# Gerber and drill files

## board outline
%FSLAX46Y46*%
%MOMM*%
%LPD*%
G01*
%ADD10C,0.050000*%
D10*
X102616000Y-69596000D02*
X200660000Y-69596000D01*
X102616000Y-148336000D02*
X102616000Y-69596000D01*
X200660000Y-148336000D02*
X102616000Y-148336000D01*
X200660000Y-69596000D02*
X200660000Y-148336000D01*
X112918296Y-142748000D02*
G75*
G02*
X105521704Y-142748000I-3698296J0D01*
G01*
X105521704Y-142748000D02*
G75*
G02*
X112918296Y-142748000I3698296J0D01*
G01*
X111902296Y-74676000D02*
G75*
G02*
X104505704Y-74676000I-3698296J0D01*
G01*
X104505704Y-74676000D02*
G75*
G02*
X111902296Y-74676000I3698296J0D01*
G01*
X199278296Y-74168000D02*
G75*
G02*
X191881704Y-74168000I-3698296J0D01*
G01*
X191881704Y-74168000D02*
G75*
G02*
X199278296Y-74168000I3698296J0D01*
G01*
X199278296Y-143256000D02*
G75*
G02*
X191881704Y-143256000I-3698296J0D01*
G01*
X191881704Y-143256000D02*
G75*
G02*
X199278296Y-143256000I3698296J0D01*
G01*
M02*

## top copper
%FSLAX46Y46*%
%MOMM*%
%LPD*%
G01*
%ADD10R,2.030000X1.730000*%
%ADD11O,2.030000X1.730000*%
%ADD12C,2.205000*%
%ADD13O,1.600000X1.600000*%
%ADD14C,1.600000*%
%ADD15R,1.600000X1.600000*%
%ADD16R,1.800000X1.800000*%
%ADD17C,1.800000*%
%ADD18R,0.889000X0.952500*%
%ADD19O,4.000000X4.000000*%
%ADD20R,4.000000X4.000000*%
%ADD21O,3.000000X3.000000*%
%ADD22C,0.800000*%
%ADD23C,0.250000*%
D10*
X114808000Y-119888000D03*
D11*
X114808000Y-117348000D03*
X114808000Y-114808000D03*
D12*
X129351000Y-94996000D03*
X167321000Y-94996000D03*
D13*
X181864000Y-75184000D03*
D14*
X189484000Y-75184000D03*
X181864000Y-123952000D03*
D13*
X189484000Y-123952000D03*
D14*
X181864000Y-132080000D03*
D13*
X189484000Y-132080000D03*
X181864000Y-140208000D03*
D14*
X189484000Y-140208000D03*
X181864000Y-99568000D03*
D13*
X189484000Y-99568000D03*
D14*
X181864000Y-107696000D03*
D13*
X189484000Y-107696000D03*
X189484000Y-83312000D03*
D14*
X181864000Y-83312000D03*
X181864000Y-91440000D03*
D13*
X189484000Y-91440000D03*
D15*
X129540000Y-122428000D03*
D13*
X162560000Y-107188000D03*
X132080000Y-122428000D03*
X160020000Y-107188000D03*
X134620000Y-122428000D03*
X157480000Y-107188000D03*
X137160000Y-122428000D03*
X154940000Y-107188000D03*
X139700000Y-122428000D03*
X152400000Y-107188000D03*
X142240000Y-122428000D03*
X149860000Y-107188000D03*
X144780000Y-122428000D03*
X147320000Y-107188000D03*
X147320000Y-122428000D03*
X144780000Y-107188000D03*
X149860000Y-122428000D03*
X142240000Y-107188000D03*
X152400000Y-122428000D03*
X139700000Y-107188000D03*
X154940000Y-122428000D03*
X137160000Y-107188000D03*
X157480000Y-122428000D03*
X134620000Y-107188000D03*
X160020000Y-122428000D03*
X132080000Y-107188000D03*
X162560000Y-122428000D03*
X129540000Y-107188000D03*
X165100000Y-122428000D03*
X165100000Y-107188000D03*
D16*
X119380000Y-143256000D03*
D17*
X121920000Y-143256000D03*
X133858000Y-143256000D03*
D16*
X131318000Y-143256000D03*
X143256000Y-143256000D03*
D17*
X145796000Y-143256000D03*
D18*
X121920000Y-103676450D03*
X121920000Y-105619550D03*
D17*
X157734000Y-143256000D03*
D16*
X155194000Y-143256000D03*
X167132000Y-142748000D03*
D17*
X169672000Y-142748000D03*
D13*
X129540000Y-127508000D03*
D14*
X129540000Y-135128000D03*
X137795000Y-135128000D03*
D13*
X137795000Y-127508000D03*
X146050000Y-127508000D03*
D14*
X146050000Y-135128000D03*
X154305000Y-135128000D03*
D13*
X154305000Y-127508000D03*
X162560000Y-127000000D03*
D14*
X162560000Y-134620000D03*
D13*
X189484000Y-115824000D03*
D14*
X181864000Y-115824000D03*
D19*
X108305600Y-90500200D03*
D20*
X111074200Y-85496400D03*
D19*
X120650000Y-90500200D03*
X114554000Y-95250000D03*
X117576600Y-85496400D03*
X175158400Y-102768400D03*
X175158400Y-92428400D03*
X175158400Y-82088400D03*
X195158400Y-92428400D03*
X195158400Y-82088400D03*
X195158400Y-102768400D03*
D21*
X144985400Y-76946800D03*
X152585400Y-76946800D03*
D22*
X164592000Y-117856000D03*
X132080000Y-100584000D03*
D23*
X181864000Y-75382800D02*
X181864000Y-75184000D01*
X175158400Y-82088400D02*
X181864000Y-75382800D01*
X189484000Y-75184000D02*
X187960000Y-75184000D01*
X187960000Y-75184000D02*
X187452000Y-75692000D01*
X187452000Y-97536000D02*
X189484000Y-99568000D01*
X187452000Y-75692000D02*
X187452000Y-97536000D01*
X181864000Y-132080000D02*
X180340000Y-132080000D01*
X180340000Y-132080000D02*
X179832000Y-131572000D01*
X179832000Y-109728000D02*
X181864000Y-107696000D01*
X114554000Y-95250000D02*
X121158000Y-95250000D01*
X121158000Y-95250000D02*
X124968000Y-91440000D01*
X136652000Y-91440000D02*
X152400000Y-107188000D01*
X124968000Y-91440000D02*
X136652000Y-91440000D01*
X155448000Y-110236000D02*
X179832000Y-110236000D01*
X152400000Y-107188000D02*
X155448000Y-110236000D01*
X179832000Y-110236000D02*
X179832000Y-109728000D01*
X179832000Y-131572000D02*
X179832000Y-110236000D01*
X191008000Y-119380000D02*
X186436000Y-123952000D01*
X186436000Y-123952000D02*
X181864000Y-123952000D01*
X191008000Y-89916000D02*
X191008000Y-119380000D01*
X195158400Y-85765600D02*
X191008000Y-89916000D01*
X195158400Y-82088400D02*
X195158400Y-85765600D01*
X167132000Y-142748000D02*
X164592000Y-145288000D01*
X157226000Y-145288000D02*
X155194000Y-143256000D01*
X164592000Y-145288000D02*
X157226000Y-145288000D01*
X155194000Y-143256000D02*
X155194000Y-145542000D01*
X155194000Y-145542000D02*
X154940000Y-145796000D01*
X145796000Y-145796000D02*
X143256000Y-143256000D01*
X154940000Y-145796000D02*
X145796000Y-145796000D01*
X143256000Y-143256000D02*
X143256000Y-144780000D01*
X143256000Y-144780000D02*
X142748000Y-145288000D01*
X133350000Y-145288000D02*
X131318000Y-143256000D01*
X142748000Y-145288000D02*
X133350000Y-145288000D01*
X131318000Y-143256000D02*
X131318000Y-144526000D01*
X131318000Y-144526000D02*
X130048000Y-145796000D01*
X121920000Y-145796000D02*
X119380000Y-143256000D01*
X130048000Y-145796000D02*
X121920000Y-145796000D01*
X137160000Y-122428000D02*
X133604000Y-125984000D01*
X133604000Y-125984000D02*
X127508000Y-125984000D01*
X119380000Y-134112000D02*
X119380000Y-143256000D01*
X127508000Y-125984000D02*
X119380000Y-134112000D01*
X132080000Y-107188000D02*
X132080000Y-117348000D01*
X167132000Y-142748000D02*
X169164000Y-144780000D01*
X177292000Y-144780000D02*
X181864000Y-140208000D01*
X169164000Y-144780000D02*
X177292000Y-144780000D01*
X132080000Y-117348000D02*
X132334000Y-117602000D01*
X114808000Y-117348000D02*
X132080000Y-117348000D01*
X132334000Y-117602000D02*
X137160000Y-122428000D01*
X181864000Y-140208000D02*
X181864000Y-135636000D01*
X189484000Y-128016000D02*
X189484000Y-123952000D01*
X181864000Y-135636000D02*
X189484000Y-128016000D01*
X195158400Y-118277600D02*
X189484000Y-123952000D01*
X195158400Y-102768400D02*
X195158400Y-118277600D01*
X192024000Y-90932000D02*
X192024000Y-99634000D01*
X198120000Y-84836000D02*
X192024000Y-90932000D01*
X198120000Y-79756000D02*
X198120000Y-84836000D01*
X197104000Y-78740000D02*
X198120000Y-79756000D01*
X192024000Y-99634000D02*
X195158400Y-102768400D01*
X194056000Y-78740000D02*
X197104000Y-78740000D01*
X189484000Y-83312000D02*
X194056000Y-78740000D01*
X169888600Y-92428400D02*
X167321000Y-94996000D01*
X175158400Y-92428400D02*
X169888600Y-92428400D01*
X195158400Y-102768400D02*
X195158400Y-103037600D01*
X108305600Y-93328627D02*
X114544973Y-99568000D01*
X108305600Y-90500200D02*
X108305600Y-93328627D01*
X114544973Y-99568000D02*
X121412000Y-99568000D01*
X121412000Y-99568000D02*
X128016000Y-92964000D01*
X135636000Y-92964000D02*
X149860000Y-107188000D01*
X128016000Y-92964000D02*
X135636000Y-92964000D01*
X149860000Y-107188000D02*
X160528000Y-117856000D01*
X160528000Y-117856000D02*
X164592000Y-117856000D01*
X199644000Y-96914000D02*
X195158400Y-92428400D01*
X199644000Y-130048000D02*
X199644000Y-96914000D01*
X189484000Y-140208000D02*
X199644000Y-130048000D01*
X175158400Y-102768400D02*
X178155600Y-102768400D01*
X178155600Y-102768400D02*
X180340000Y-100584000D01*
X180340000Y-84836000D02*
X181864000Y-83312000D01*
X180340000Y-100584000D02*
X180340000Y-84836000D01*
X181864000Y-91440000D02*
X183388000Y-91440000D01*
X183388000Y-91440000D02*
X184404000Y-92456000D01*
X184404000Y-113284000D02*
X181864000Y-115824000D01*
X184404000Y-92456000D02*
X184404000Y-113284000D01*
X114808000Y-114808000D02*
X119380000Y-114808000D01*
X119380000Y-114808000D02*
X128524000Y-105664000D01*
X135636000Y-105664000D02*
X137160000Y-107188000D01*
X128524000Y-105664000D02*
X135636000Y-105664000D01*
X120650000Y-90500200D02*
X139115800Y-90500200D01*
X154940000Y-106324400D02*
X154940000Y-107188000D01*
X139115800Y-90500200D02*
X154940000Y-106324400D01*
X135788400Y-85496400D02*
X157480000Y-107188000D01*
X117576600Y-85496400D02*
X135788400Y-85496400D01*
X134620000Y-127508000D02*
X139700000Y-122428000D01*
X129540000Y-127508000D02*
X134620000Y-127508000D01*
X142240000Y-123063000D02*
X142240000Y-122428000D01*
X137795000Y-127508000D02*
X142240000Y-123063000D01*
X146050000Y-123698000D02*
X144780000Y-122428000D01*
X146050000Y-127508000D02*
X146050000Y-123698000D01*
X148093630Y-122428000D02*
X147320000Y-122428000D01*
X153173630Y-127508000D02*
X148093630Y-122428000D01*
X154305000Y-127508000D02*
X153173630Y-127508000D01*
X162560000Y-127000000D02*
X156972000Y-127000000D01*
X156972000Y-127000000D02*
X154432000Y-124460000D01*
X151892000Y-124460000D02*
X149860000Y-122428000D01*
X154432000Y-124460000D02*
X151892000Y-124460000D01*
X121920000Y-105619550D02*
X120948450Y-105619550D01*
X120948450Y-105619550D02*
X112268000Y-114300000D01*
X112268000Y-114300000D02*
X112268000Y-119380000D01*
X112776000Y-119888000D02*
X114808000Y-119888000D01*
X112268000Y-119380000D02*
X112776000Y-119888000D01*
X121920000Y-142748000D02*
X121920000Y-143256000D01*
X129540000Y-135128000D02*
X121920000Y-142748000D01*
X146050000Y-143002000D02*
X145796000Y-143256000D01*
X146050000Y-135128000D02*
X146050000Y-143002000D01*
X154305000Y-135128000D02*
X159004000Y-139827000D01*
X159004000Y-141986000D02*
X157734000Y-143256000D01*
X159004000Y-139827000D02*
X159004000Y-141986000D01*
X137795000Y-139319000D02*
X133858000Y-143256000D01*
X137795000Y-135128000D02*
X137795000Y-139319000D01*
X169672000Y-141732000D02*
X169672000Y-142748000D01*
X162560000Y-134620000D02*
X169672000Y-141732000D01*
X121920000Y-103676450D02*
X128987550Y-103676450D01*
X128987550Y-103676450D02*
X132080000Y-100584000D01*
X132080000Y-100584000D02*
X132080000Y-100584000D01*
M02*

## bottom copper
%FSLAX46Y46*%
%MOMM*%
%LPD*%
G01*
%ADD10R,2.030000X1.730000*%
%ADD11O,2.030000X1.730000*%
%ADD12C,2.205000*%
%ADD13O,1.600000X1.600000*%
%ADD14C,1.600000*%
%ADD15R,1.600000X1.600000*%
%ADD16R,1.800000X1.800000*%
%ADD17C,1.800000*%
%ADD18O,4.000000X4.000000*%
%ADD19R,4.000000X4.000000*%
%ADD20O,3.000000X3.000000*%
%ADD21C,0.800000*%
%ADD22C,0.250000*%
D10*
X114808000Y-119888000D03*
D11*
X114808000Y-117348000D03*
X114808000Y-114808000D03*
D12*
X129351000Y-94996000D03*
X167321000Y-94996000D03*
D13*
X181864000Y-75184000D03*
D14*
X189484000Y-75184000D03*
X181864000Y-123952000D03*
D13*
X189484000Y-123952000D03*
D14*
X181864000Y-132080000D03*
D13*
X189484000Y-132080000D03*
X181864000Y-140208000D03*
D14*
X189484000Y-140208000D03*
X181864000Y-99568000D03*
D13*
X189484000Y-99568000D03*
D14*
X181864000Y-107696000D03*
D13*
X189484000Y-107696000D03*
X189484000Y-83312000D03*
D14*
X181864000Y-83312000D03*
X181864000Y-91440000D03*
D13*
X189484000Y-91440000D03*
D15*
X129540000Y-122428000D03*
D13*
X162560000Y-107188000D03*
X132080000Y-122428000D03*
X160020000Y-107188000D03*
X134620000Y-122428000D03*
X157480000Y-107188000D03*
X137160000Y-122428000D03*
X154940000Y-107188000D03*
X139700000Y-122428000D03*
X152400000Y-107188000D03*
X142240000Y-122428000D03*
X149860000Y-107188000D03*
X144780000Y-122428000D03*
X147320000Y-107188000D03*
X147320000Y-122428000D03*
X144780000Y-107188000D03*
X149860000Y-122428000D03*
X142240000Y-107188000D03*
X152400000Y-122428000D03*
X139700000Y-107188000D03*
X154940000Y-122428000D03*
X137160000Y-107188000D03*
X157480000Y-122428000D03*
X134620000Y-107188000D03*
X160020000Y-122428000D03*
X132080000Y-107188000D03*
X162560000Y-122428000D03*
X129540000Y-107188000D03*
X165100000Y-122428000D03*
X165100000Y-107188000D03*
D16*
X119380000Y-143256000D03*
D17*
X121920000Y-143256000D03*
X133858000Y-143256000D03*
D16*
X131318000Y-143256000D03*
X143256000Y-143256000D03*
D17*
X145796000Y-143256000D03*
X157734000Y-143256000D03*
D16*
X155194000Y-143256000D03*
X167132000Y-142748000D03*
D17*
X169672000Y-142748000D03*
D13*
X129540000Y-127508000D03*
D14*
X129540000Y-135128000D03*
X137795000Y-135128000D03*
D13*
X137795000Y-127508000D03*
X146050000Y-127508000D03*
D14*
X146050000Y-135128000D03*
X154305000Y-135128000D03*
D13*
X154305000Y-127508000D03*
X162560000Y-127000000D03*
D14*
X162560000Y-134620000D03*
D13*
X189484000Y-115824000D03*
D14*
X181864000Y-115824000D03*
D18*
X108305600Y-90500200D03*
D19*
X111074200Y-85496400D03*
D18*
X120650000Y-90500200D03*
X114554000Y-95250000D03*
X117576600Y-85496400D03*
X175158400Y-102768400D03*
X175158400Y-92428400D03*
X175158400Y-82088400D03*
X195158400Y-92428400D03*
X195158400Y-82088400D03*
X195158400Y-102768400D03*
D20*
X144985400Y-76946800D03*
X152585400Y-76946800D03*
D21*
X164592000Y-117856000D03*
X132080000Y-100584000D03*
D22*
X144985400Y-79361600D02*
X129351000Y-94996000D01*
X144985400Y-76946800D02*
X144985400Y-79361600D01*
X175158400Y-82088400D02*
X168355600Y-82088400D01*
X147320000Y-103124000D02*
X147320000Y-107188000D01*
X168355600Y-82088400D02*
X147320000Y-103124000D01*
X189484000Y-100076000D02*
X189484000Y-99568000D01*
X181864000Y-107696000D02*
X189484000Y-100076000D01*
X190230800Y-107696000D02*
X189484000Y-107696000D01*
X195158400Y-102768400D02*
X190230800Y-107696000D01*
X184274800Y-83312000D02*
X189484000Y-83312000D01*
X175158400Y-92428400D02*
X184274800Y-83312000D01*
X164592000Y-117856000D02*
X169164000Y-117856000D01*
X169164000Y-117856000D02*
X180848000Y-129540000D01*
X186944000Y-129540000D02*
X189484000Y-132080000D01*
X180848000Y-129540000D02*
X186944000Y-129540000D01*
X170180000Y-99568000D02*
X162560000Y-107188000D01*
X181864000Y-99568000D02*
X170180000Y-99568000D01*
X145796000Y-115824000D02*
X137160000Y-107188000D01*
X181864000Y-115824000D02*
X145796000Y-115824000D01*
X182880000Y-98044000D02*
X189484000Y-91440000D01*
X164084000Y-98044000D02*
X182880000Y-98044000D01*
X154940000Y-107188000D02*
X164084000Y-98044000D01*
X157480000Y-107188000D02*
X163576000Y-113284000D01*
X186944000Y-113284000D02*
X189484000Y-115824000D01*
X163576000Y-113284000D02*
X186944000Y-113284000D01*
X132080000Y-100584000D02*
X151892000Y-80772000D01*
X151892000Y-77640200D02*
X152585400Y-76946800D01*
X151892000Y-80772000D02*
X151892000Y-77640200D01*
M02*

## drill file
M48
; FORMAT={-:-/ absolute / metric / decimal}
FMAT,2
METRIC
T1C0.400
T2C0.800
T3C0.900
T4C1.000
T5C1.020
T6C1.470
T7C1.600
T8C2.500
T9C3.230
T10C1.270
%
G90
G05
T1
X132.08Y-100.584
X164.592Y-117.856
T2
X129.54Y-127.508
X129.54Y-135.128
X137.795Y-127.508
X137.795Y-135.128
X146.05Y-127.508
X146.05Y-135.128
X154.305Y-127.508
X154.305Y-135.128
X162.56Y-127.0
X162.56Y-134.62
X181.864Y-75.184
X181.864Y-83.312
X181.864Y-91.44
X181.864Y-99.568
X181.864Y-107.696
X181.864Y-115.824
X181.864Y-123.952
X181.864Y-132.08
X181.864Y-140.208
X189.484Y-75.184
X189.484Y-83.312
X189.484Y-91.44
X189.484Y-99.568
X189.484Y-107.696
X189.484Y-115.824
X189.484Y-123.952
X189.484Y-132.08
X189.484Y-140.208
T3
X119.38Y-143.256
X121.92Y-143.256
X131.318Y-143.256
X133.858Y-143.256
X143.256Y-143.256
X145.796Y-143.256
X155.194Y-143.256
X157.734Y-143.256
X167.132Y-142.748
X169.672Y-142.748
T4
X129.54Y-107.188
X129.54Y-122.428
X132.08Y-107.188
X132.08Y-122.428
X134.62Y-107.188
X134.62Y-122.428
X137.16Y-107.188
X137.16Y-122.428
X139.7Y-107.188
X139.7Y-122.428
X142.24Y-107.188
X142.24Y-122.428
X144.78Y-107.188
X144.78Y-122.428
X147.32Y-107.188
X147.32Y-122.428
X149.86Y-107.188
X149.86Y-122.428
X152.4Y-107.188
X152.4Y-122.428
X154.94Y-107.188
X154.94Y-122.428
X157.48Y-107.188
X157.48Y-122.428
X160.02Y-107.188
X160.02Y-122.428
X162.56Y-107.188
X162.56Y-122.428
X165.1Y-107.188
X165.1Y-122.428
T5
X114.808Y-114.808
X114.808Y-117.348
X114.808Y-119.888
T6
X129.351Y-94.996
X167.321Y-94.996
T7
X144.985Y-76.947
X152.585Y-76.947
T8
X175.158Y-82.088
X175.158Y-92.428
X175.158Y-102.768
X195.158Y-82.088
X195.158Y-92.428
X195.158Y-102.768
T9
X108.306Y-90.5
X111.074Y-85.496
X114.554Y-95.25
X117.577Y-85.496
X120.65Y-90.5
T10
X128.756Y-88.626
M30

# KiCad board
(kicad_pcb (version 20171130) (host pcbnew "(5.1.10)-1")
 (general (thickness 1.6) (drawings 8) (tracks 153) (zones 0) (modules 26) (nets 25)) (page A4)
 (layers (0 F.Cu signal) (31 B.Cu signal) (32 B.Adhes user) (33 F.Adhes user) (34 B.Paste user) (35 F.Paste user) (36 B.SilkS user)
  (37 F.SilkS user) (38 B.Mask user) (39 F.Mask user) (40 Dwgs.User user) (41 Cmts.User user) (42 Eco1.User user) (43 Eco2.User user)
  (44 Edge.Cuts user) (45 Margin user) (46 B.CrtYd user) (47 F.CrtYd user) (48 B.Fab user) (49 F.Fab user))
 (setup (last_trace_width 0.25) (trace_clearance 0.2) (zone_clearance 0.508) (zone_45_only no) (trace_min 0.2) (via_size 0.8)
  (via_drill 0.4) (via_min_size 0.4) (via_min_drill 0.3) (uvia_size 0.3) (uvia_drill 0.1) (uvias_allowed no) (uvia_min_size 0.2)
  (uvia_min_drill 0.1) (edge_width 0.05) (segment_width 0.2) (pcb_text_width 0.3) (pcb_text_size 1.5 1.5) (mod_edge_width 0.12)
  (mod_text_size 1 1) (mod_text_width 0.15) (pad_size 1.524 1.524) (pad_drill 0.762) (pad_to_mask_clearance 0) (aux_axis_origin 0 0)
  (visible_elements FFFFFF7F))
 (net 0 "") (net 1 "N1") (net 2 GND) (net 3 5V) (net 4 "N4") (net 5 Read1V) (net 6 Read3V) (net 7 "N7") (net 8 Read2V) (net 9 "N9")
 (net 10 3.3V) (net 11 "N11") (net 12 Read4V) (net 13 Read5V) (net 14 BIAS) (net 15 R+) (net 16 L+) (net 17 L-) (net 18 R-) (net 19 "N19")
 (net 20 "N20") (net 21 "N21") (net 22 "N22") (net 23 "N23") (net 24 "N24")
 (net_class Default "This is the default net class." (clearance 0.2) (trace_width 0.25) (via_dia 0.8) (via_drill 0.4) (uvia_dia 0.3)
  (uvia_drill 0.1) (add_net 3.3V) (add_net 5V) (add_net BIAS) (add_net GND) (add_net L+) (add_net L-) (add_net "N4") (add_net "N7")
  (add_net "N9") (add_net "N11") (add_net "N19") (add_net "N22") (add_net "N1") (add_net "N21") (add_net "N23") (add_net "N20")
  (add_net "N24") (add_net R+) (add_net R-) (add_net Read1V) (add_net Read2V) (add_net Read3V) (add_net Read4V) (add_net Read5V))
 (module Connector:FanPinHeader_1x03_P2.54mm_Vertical (layer F.Cu) (at 114.808 119.888 90)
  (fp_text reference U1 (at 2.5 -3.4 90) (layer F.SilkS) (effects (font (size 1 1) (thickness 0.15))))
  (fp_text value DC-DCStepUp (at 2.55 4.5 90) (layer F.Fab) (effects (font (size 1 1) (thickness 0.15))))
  (pad 1 thru_hole rect (at 0 0 180) (size 2.03 1.73) (drill 1.02) (layers *.Cu *.Mask) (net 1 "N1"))
  (pad 3 thru_hole oval (at 2.54 0 180) (size 2.03 1.73) (drill 1.02) (layers *.Cu *.Mask) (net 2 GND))
  (pad 2 thru_hole oval (at 5.08 0 180) (size 2.03 1.73) (drill 1.02) (layers *.Cu *.Mask) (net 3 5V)))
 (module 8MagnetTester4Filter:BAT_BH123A (layer F.Cu) (at 148.336 94.996 180)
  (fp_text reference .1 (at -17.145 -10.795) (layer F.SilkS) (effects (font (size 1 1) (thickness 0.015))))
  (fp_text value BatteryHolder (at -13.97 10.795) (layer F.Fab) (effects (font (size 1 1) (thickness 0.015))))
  (pad None np_thru_hole circle (at 19.58 6.37 180) (size 1.27 1.27) (drill 1.27) (layers *.Cu *.Mask))
  (pad 2 thru_hole circle (at 18.985 0 180) (size 2.205 2.205) (drill 1.47) (layers *.Cu *.Mask) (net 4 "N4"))
  (pad 1 thru_hole circle (at -18.985 0 180) (size 2.205 2.205) (drill 1.47) (layers *.Cu *.Mask) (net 2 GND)))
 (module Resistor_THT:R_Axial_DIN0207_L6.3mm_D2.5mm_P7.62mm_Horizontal (layer F.Cu) (at 189.484 75.184 180)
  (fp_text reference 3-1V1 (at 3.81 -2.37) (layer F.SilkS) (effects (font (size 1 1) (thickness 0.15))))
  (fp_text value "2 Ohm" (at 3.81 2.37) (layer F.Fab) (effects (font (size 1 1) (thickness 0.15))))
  (pad 2 thru_hole oval (at 7.62 0 180) (size 1.6 1.6) (drill 0.8) (layers *.Cu *.Mask) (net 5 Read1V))
  (pad 1 thru_hole circle (at 0 0 180) (size 1.6 1.6) (drill 0.8) (layers *.Cu *.Mask) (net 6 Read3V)))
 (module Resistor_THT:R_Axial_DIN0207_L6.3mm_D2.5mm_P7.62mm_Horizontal (layer F.Cu) (at 181.864 123.952)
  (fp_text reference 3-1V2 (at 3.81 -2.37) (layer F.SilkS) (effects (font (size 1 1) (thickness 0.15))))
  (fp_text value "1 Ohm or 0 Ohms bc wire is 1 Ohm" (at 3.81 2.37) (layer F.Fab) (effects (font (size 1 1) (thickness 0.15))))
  (pad 1 thru_hole circle (at 0 0) (size 1.6 1.6) (drill 0.8) (layers *.Cu *.Mask) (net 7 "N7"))
  (pad 2 thru_hole oval (at 7.62 0) (size 1.6 1.6) (drill 0.8) (layers *.Cu *.Mask) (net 2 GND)))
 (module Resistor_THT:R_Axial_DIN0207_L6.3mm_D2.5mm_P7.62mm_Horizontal (layer F.Cu) (at 181.864 132.08)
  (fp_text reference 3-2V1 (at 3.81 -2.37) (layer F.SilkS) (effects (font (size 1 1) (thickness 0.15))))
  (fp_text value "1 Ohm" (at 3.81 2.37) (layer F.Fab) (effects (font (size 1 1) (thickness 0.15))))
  (pad 1 thru_hole circle (at 0 0) (size 1.6 1.6) (drill 0.8) (layers *.Cu *.Mask) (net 6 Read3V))
  (pad 2 thru_hole oval (at 7.62 0) (size 1.6 1.6) (drill 0.8) (layers *.Cu *.Mask) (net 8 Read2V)))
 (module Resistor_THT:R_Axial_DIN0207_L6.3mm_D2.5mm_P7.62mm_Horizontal (layer F.Cu) (at 189.484 140.208 180)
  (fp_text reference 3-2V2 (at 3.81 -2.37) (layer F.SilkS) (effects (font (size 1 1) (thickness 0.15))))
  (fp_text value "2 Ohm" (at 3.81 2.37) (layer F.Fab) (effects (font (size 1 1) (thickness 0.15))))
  (pad 2 thru_hole oval (at 7.62 0 180) (size 1.6 1.6) (drill 0.8) (layers *.Cu *.Mask) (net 2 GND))
  (pad 1 thru_hole circle (at 0 0 180) (size 1.6 1.6) (drill 0.8) (layers *.Cu *.Mask) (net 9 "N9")))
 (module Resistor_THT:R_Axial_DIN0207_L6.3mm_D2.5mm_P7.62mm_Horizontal (layer F.Cu) (at 181.864 99.568)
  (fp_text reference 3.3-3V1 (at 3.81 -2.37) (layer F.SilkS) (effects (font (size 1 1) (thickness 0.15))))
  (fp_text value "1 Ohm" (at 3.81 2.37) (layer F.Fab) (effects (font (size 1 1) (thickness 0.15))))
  (pad 1 thru_hole circle (at 0 0) (size 1.6 1.6) (drill 0.8) (layers *.Cu *.Mask) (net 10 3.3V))
  (pad 2 thru_hole oval (at 7.62 0) (size 1.6 1.6) (drill 0.8) (layers *.Cu *.Mask) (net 6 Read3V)))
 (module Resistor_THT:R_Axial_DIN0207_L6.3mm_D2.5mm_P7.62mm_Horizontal (layer F.Cu) (at 181.864 107.696)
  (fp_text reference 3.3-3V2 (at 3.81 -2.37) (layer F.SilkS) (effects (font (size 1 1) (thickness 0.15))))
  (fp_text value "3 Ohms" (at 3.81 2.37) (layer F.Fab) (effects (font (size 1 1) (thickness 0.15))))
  (pad 1 thru_hole circle (at 0 0) (size 1.6 1.6) (drill 0.8) (layers *.Cu *.Mask) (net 6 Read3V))
  (pad 2 thru_hole oval (at 7.62 0) (size 1.6 1.6) (drill 0.8) (layers *.Cu *.Mask) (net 2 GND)))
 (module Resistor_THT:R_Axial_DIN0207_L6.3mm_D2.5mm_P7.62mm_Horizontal (layer F.Cu) (at 181.864 83.312)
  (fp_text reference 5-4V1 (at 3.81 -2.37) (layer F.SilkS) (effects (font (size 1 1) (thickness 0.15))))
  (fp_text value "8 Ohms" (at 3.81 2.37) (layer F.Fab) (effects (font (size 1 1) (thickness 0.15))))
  (pad 2 thru_hole oval (at 7.62 0) (size 1.6 1.6) (drill 0.8) (layers *.Cu *.Mask) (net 2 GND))
  (pad 1 thru_hole circle (at 0 0) (size 1.6 1.6) (drill 0.8) (layers *.Cu *.Mask) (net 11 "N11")))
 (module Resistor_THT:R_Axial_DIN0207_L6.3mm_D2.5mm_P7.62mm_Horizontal (layer F.Cu) (at 181.864 91.44)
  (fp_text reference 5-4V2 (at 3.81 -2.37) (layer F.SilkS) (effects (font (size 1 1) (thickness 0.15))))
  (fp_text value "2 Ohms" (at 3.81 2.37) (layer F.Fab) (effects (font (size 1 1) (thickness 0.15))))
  (pad 1 thru_hole circle (at 0 0) (size 1.6 1.6) (drill 0.8) (layers *.Cu *.Mask) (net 3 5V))
  (pad 2 thru_hole oval (at 7.62 0) (size 1.6 1.6) (drill 0.8) (layers *.Cu *.Mask) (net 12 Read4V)))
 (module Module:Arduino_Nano (layer F.Cu) (at 129.54 122.428 90)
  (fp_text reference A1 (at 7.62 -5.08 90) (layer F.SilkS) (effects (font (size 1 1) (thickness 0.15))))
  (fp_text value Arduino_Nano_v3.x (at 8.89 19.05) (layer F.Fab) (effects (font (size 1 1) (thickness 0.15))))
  (pad 1 thru_hole rect (at 0 0 90) (size 1.6 1.6) (drill 1) (layers *.Cu *.Mask))
  (pad 17 thru_hole oval (at 15.24 33.02 90) (size 1.6 1.6) (drill 1) (layers *.Cu *.Mask) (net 10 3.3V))
  (pad 2 thru_hole oval (at 0 2.54 90) (size 1.6 1.6) (drill 1) (layers *.Cu *.Mask))
  (pad 18 thru_hole oval (at 15.24 30.48 90) (size 1.6 1.6) (drill 1) (layers *.Cu *.Mask))
  (pad 3 thru_hole oval (at 0 5.08 90) (size 1.6 1.6) (drill 1) (layers *.Cu *.Mask))
  (pad 19 thru_hole oval (at 15.24 27.94 90) (size 1.6 1.6) (drill 1) (layers *.Cu *.Mask) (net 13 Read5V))
  (pad 4 thru_hole oval (at 0 7.62 90) (size 1.6 1.6) (drill 1) (layers *.Cu *.Mask) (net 2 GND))
  (pad 20 thru_hole oval (at 15.24 25.4 90) (size 1.6 1.6) (drill 1) (layers *.Cu *.Mask) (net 12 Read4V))
  (pad 5 thru_hole oval (at 0 10.16 90) (size 1.6 1.6) (drill 1) (layers *.Cu *.Mask) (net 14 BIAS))
  (pad 21 thru_hole oval (at 15.24 22.86 90) (size 1.6 1.6) (drill 1) (layers *.Cu *.Mask) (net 6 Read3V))
  (pad 6 thru_hole oval (at 0 12.7 90) (size 1.6 1.6) (drill 1) (layers *.Cu *.Mask) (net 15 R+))
  (pad 22 thru_hole oval (at 15.24 20.32 90) (size 1.6 1.6) (drill 1) (layers *.Cu *.Mask) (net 8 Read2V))
  (pad 7 thru_hole oval (at 0 15.24 90) (size 1.6 1.6) (drill 1) (layers *.Cu *.Mask) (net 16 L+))
  (pad 23 thru_hole oval (at 15.24 17.78 90) (size 1.6 1.6) (drill 1) (layers *.Cu *.Mask) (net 5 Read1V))
  (pad 8 thru_hole oval (at 0 17.78 90) (size 1.6 1.6) (drill 1) (layers *.Cu *.Mask) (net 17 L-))
  (pad 24 thru_hole oval (at 15.24 15.24 90) (size 1.6 1.6) (drill 1) (layers *.Cu *.Mask))
  (pad 9 thru_hole oval (at 0 20.32 90) (size 1.6 1.6) (drill 1) (layers *.Cu *.Mask) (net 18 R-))
  (pad 25 thru_hole oval (at 15.24 12.7 90) (size 1.6 1.6) (drill 1) (layers *.Cu *.Mask))
  (pad 10 thru_hole oval (at 0 22.86 90) (size 1.6 1.6) (drill 1) (layers *.Cu *.Mask))
  (pad 26 thru_hole oval (at 15.24 10.16 90) (size 1.6 1.6) (drill 1) (layers *.Cu *.Mask))
  (pad 11 thru_hole oval (at 0 25.4 90) (size 1.6 1.6) (drill 1) (layers *.Cu *.Mask))
  (pad 27 thru_hole oval (at 15.24 7.62 90) (size 1.6 1.6) (drill 1) (layers *.Cu *.Mask) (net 3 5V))
  (pad 12 thru_hole oval (at 0 27.94 90) (size 1.6 1.6) (drill 1) (layers *.Cu *.Mask))
  (pad 28 thru_hole oval (at 15.24 5.08 90) (size 1.6 1.6) (drill 1) (layers *.Cu *.Mask))
  (pad 13 thru_hole oval (at 0 30.48 90) (size 1.6 1.6) (drill 1) (layers *.Cu *.Mask))
  (pad 29 thru_hole oval (at 15.24 2.54 90) (size 1.6 1.6) (drill 1) (layers *.Cu *.Mask) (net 2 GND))
  (pad 14 thru_hole oval (at 0 33.02 90) (size 1.6 1.6) (drill 1) (layers *.Cu *.Mask))
  (pad 30 thru_hole oval (at 15.24 0 90) (size 1.6 1.6) (drill 1) (layers *.Cu *.Mask))
  (pad 15 thru_hole oval (at 0 35.56 90) (size 1.6 1.6) (drill 1) (layers *.Cu *.Mask))
  (pad 16 thru_hole oval (at 15.24 35.56 90) (size 1.6 1.6) (drill 1) (layers *.Cu *.Mask)))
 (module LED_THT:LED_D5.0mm (layer F.Cu) (at 119.38 143.256)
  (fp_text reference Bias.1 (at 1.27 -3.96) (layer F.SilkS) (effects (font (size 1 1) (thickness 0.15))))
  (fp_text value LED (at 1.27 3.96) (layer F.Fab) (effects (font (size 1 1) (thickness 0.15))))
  (pad 1 thru_hole rect (at 0 0) (size 1.8 1.8) (drill 0.9) (layers *.Cu *.Mask) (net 2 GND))
  (pad 2 thru_hole circle (at 2.54 0) (size 1.8 1.8) (drill 0.9) (layers *.Cu *.Mask) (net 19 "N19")))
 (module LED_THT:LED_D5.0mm (layer F.Cu) (at 131.318 143.256)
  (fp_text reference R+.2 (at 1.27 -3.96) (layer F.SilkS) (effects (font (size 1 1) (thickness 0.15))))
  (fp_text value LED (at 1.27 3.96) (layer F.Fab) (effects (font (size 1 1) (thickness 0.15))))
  (pad 2 thru_hole circle (at 2.54 0) (size 1.8 1.8) (drill 0.9) (layers *.Cu *.Mask) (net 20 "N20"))
  (pad 1 thru_hole rect (at 0 0) (size 1.8 1.8) (drill 0.9) (layers *.Cu *.Mask) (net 2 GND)))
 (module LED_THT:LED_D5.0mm (layer F.Cu) (at 143.256 143.256)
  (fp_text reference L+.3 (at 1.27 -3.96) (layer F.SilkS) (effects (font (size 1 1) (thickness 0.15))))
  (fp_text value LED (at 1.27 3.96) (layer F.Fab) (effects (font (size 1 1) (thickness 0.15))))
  (pad 1 thru_hole rect (at 0 0) (size 1.8 1.8) (drill 0.9) (layers *.Cu *.Mask) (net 2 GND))
  (pad 2 thru_hole circle (at 2.54 0) (size 1.8 1.8) (drill 0.9) (layers *.Cu *.Mask) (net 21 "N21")))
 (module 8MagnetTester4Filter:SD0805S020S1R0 (layer F.Cu) (at 121.92 104.648 270)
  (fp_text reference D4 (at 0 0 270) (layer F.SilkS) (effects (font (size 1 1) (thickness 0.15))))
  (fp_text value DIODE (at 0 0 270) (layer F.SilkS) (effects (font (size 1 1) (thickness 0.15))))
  (pad 1 smd rect (at -0.97155 0 270) (size 0.9525 0.889) (layers F.Cu F.Paste F.Mask) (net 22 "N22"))
  (pad 2 smd rect (at 0.97155 0 270) (size 0.9525 0.889) (layers F.Cu F.Paste F.Mask) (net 1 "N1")))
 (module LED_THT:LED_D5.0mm (layer F.Cu) (at 155.194 143.256)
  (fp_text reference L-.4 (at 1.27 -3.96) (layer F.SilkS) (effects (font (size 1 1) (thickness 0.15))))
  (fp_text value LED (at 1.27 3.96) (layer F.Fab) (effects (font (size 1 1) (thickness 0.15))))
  (pad 2 thru_hole circle (at 2.54 0) (size 1.8 1.8) (drill 0.9) (layers *.Cu *.Mask) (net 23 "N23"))
  (pad 1 thru_hole rect (at 0 0) (size 1.8 1.8) (drill 0.9) (layers *.Cu *.Mask) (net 2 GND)))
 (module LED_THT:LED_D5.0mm (layer F.Cu) (at 167.132 142.748)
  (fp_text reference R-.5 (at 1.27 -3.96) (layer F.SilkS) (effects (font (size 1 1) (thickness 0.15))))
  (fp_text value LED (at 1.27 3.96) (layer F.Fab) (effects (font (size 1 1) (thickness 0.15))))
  (pad 1 thru_hole rect (at 0 0) (size 1.8 1.8) (drill 0.9) (layers *.Cu *.Mask) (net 2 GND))
  (pad 2 thru_hole circle (at 2.54 0) (size 1.8 1.8) (drill 0.9) (layers *.Cu *.Mask) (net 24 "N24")))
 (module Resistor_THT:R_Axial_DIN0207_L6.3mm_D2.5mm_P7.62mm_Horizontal (layer F.Cu) (at 129.54 135.128 90)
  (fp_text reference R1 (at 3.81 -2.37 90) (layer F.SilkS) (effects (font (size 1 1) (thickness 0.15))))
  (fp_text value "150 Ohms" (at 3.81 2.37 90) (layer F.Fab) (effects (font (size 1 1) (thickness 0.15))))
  (pad 2 thru_hole oval (at 7.62 0 90) (size 1.6 1.6) (drill 0.8) (layers *.Cu *.Mask) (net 14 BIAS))
  (pad 1 thru_hole circle (at 0 0 90) (size 1.6 1.6) (drill 0.8) (layers *.Cu *.Mask) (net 19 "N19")))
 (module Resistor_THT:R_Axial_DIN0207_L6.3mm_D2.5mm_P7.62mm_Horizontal (layer F.Cu) (at 137.795 135.128 90)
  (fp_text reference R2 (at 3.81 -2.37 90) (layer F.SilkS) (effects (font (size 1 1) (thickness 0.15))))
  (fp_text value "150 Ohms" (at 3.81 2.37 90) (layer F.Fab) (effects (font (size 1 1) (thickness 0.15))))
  (pad 1 thru_hole circle (at 0 0 90) (size 1.6 1.6) (drill 0.8) (layers *.Cu *.Mask) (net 20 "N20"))
  (pad 2 thru_hole oval (at 7.62 0 90) (size 1.6 1.6) (drill 0.8) (layers *.Cu *.Mask) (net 15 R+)))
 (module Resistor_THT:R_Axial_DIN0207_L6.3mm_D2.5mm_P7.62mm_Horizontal (layer F.Cu) (at 146.05 135.128 90)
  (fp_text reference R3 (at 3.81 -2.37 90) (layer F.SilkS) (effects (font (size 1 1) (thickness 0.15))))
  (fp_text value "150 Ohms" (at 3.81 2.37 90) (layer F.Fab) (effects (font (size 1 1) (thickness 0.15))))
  (pad 2 thru_hole oval (at 7.62 0 90) (size 1.6 1.6) (drill 0.8) (layers *.Cu *.Mask) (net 16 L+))
  (pad 1 thru_hole circle (at 0 0 90) (size 1.6 1.6) (drill 0.8) (layers *.Cu *.Mask) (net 21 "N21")))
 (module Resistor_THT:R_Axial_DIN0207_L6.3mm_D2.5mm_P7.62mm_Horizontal (layer F.Cu) (at 154.305 135.128 90)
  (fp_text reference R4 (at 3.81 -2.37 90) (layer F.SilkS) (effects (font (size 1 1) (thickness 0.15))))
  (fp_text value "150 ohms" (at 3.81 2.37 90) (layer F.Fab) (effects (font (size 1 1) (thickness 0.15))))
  (pad 1 thru_hole circle (at 0 0 90) (size 1.6 1.6) (drill 0.8) (layers *.Cu *.Mask) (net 23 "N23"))
  (pad 2 thru_hole oval (at 7.62 0 90) (size 1.6 1.6) (drill 0.8) (layers *.Cu *.Mask) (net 17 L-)))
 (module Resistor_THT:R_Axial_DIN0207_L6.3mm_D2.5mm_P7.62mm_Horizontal (layer F.Cu) (at 162.56 134.62 90)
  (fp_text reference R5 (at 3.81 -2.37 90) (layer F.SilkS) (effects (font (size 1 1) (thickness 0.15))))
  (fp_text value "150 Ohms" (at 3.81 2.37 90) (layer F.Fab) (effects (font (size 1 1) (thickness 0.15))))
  (pad 2 thru_hole oval (at 7.62 0 90) (size 1.6 1.6) (drill 0.8) (layers *.Cu *.Mask) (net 18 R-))
  (pad 1 thru_hole circle (at 0 0 90) (size 1.6 1.6) (drill 0.8) (layers *.Cu *.Mask) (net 24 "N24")))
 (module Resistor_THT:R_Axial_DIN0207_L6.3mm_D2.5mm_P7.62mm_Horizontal (layer F.Cu) (at 181.864 115.824)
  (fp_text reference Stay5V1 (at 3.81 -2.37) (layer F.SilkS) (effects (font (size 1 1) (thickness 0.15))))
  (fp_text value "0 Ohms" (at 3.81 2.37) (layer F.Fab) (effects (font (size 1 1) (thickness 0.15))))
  (pad 2 thru_hole oval (at 7.62 0) (size 1.6 1.6) (drill 0.8) (layers *.Cu *.Mask) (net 13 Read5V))
  (pad 1 thru_hole circle (at 0 0) (size 1.6 1.6) (drill 0.8) (layers *.Cu *.Mask) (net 3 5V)))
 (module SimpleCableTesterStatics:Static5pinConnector (layer F.Cu) (at 114.3 86.36)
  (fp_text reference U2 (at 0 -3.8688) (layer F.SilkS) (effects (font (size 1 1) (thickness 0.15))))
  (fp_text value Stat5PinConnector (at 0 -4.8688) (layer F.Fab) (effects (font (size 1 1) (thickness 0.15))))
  (pad 2 thru_hole oval (at -5.9944 4.1402) (size 4 4) (drill 3.23) (layers *.Cu *.Mask) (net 8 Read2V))
  (pad 1 thru_hole rect (at -3.2258 -0.8636) (size 4 4) (drill 3.23) (layers *.Cu *.Mask))
  (pad 4 thru_hole oval (at 6.35 4.1402) (size 4 4) (drill 3.23) (layers *.Cu *.Mask) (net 12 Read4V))
  (pad 3 thru_hole oval (at 0.254 8.89) (size 4 4) (drill 3.23) (layers *.Cu *.Mask) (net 6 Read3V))
  (pad 5 thru_hole oval (at 3.2766 -0.8636) (size 4 4) (drill 3.23) (layers *.Cu *.Mask) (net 13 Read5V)))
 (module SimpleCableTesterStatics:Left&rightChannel (layer F.Cu) (at 170.18 97.028 90)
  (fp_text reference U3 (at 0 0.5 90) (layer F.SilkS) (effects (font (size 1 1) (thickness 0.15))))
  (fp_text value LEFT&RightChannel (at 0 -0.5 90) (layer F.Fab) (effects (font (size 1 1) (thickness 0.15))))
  (pad 4 thru_hole oval (at -5.7404 4.9784 90) (size 4 4) (drill 2.5) (layers *.Cu *.Mask) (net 11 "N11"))
  (pad 3 thru_hole oval (at 4.5996 4.9784 90) (size 4 4) (drill 2.5) (layers *.Cu *.Mask) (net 2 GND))
  (pad 1L thru_hole oval (at 14.9396 4.9784 90) (size 4 4) (drill 2.5) (layers *.Cu *.Mask) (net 5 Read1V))
  (pad 2 thru_hole oval (at 4.5996 24.9784 90) (size 4 4) (drill 2.5) (layers *.Cu *.Mask) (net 9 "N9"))
  (pad 1R thru_hole oval (at 14.9396 24.9784 90) (size 4 4) (drill 2.5) (layers *.Cu *.Mask) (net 7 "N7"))
  (pad 5 thru_hole oval (at -5.7404 24.9784 90) (size 4 4) (drill 2.5) (layers *.Cu *.Mask) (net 2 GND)))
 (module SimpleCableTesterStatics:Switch (layer F.Cu) (at 148.844 73.152)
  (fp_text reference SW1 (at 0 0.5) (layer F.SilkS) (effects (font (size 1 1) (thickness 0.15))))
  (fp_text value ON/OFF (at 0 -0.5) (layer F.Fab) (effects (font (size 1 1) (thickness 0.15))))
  (pad 1 thru_hole oval (at -3.8586 3.7948) (size 3 3) (drill 1.6) (layers *.Cu *.Mask) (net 4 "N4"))
  (pad 2 thru_hole oval (at 3.7414 3.7948) (size 3 3) (drill 1.6) (layers *.Cu *.Mask) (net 22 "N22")))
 (gr_line (start 102.616 69.596) (end 200.66 69.596) (layer Edge.Cuts) (width 0.05))
 (gr_line (start 102.616 148.336) (end 102.616 69.596) (layer Edge.Cuts) (width 0.05))
 (gr_line (start 200.66 148.336) (end 102.616 148.336) (layer Edge.Cuts) (width 0.05))
 (gr_line (start 200.66 69.596) (end 200.66 148.336) (layer Edge.Cuts) (width 0.05))
 (gr_circle (center 109.22 142.748) (end 112.776 143.764) (layer Edge.Cuts) (width 0.05))
 (gr_circle (center 108.204 74.676) (end 111.76 75.692) (layer Edge.Cuts) (width 0.05))
 (gr_circle (center 195.58 74.168) (end 199.136 75.184) (layer Edge.Cuts) (width 0.05))
 (gr_circle (center 195.58 143.256) (end 199.136 144.272) (layer Edge.Cuts) (width 0.05))
 (segment (start 144.9854 79.3616) (end 129.351 94.996) (width 0.25) (layer B.Cu) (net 4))
 (segment (start 144.9854 76.9468) (end 144.9854 79.3616) (width 0.25) (layer B.Cu) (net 4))
 (segment (start 181.864 75.3828) (end 181.864 75.184) (width 0.25) (layer F.Cu) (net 5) (status 30))
 (segment (start 175.1584 82.0884) (end 181.864 75.3828) (width 0.25) (layer F.Cu) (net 5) (status 30))
 (segment (start 175.1584 82.0884) (end 168.3556 82.0884) (width 0.25) (layer B.Cu) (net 5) (status 10))
 (segment (start 147.32 103.124) (end 147.32 107.188) (width 0.25) (layer B.Cu) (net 5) (status 20))
 (segment (start 168.3556 82.0884) (end 147.32 103.124) (width 0.25) (layer B.Cu) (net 5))
 (segment (start 189.484 75.184) (end 187.96 75.184) (width 0.25) (layer F.Cu) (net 6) (status 10))
 (segment (start 187.96 75.184) (end 187.452 75.692) (width 0.25) (layer F.Cu) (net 6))
 (segment (start 187.452 97.536) (end 189.484 99.568) (width 0.25) (layer F.Cu) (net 6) (status 20))
 (segment (start 187.452 75.692) (end 187.452 97.536) (width 0.25) (layer F.Cu) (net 6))
 (segment (start 181.864 132.08) (end 180.34 132.08) (width 0.25) (layer F.Cu) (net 6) (status 10))
 (segment (start 180.34 132.08) (end 179.832 131.572) (width 0.25) (layer F.Cu) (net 6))
 (segment (start 179.832 109.728) (end 181.864 107.696) (width 0.25) (layer F.Cu) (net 6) (status 20))
 (segment (start 189.484 100.076) (end 189.484 99.568) (width 0.25) (layer B.Cu) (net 6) (status 30))
 (segment (start 181.864 107.696) (end 189.484 100.076) (width 0.25) (layer B.Cu) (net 6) (status 30))
 (segment (start 114.554 95.25) (end 121.158 95.25) (width 0.25) (layer F.Cu) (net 6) (status 10))
 (segment (start 121.158 95.25) (end 124.968 91.44) (width 0.25) (layer F.Cu) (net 6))
 (segment (start 136.652 91.44) (end 152.4 107.188) (width 0.25) (layer F.Cu) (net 6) (status 20))
 (segment (start 124.968 91.44) (end 136.652 91.44) (width 0.25) (layer F.Cu) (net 6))
 (segment (start 155.448 110.236) (end 179.832 110.236) (width 0.25) (layer F.Cu) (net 6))
 (segment (start 152.4 107.188) (end 155.448 110.236) (width 0.25) (layer F.Cu) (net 6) (status 10))
 (segment (start 179.832 110.236) (end 179.832 109.728) (width 0.25) (layer F.Cu) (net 6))
 (segment (start 179.832 131.572) (end 179.832 110.236) (width 0.25) (layer F.Cu) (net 6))
 (segment (start 191.008 119.38) (end 186.436 123.952) (width 0.25) (layer F.Cu) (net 7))
 (segment (start 186.436 123.952) (end 181.864 123.952) (width 0.25) (layer F.Cu) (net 7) (status 20))
 (segment (start 191.008 89.916) (end 191.008 119.38) (width 0.25) (layer F.Cu) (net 7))
 (segment (start 195.1584 85.7656) (end 191.008 89.916) (width 0.25) (layer F.Cu) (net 7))
 (segment (start 195.1584 82.0884) (end 195.1584 85.7656) (width 0.25) (layer F.Cu) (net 7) (status 10))
 (segment (start 167.132 142.748) (end 164.592 145.288) (width 0.25) (layer F.Cu) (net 2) (status 10))
 (segment (start 157.226 145.288) (end 155.194 143.256) (width 0.25) (layer F.Cu) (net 2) (status 20))
 (segment (start 164.592 145.288) (end 157.226 145.288) (width 0.25) (layer F.Cu) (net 2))
 (segment (start 155.194 143.256) (end 155.194 145.542) (width 0.25) (layer F.Cu) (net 2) (status 10))
 (segment (start 155.194 145.542) (end 154.94 145.796) (width 0.25) (layer F.Cu) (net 2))
 (segment (start 145.796 145.796) (end 143.256 143.256) (width 0.25) (layer F.Cu) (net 2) (status 20))
 (segment (start 154.94 145.796) (end 145.796 145.796) (width 0.25) (layer F.Cu) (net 2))
 (segment (start 143.256 143.256) (end 143.256 144.78) (width 0.25) (layer F.Cu) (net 2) (status 10))
 (segment (start 143.256 144.78) (end 142.748 145.288) (width 0.25) (layer F.Cu) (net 2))
 (segment (start 133.35 145.288) (end 131.318 143.256) (width 0.25) (layer F.Cu) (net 2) (status 20))
 (segment (start 142.748 145.288) (end 133.35 145.288) (width 0.25) (layer F.Cu) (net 2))
 (segment (start 131.318 143.256) (end 131.318 144.526) (width 0.25) (layer F.Cu) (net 2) (status 10))
 (segment (start 131.318 144.526) (end 130.048 145.796) (width 0.25) (layer F.Cu) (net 2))
 (segment (start 121.92 145.796) (end 119.38 143.256) (width 0.25) (layer F.Cu) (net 2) (status 20))
 (segment (start 130.048 145.796) (end 121.92 145.796) (width 0.25) (layer F.Cu) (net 2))
 (segment (start 137.16 122.428) (end 133.604 125.984) (width 0.25) (layer F.Cu) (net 2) (status 10))
 (segment (start 133.604 125.984) (end 127.508 125.984) (width 0.25) (layer F.Cu) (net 2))
 (segment (start 119.38 134.112) (end 119.38 143.256) (width 0.25) (layer F.Cu) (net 2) (status 20))
 (segment (start 127.508 125.984) (end 119.38 134.112) (width 0.25) (layer F.Cu) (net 2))
 (segment (start 132.08 107.188) (end 132.08 117.348) (width 0.25) (layer F.Cu) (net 2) (status 10))
 (segment (start 167.132 142.748) (end 169.164 144.78) (width 0.25) (layer F.Cu) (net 2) (status 10))
 (segment (start 177.292 144.78) (end 181.864 140.208) (width 0.25) (layer F.Cu) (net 2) (status 20))
 (segment (start 169.164 144.78) (end 177.292 144.78) (width 0.25) (layer F.Cu) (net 2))
 (segment (start 132.08 117.348) (end 132.334 117.602) (width 0.25) (layer F.Cu) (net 2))
 (segment (start 114.808 117.348) (end 132.08 117.348) (width 0.25) (layer F.Cu) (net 2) (status 10))
 (segment (start 132.334 117.602) (end 137.16 122.428) (width 0.25) (layer F.Cu) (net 2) (status 20))
 (segment (start 181.864 140.208) (end 181.864 135.636) (width 0.25) (layer F.Cu) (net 2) (status 10))
 (segment (start 189.484 128.016) (end 189.484 123.952) (width 0.25) (layer F.Cu) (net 2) (status 20))
 (segment (start 181.864 135.636) (end 189.484 128.016) (width 0.25) (layer F.Cu) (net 2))
 (segment (start 195.1584 118.2776) (end 189.484 123.952) (width 0.25) (layer F.Cu) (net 2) (status 20))
 (segment (start 195.1584 102.7684) (end 195.1584 118.2776) (width 0.25) (layer F.Cu) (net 2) (status 10))
 (segment (start 192.024 90.932) (end 192.024 99.634) (width 0.25) (layer F.Cu) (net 2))
 (segment (start 198.12 84.836) (end 192.024 90.932) (width 0.25) (layer F.Cu) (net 2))
 (segment (start 198.12 79.756) (end 198.12 84.836) (width 0.25) (layer F.Cu) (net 2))
 (segment (start 197.104 78.74) (end 198.12 79.756) (width 0.25) (layer F.Cu) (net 2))
 (segment (start 192.024 99.634) (end 195.1584 102.7684) (width 0.25) (layer F.Cu) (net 2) (status 20))
 (segment (start 194.056 78.74) (end 197.104 78.74) (width 0.25) (layer F.Cu) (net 2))
 (segment (start 189.484 83.312) (end 194.056 78.74) (width 0.25) (layer F.Cu) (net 2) (status 10))
 (segment (start 169.8886 92.4284) (end 167.321 94.996) (width 0.25) (layer F.Cu) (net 2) (status 20))
 (segment (start 175.1584 92.4284) (end 169.8886 92.4284) (width 0.25) (layer F.Cu) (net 2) (status 10))
 (segment (start 195.1584 102.7684) (end 195.1584 103.0376) (width 0.25) (layer F.Cu) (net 2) (status 30))
 (segment (start 190.2308 107.696) (end 189.484 107.696) (width 0.25) (layer B.Cu) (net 2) (status 30))
 (segment (start 195.1584 102.7684) (end 190.2308 107.696) (width 0.25) (layer B.Cu) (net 2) (status 30))
 (segment (start 184.2748 83.312) (end 189.484 83.312) (width 0.25) (layer B.Cu) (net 2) (status 20))
 (segment (start 175.1584 92.4284) (end 184.2748 83.312) (width 0.25) (layer B.Cu) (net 2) (status 10))
 (segment (start 108.3056 93.328627) (end 114.544973 99.568) (width 0.25) (layer F.Cu) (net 8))
 (segment (start 108.3056 90.5002) (end 108.3056 93.328627) (width 0.25) (layer F.Cu) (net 8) (status 10))
 (segment (start 114.544973 99.568) (end 121.412 99.568) (width 0.25) (layer F.Cu) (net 8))
 (segment (start 121.412 99.568) (end 128.016 92.964) (width 0.25) (layer F.Cu) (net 8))
 (segment (start 135.636 92.964) (end 149.86 107.188) (width 0.25) (layer F.Cu) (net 8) (status 20))
 (segment (start 128.016 92.964) (end 135.636 92.964) (width 0.25) (layer F.Cu) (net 8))
 (segment (start 149.86 107.188) (end 160.528 117.856) (width 0.25) (layer F.Cu) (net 8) (status 10))
 (segment (start 160.528 117.856) (end 164.592 117.856) (width 0.25) (layer F.Cu) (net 8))
 (via (at 164.592 117.856) (size 0.8) (drill 0.4) (layers F.Cu B.Cu) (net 8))
 (segment (start 164.592 117.856) (end 169.164 117.856) (width 0.25) (layer B.Cu) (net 8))
 (segment (start 169.164 117.856) (end 180.848 129.54) (width 0.25) (layer B.Cu) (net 8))
 (segment (start 186.944 129.54) (end 189.484 132.08) (width 0.25) (layer B.Cu) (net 8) (status 20))
 (segment (start 180.848 129.54) (end 186.944 129.54) (width 0.25) (layer B.Cu) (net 8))
 (segment (start 199.644 96.914) (end 195.1584 92.4284) (width 0.25) (layer F.Cu) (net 9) (status 20))
 (segment (start 199.644 130.048) (end 199.644 96.914) (width 0.25) (layer F.Cu) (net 9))
 (segment (start 189.484 140.208) (end 199.644 130.048) (width 0.25) (layer F.Cu) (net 9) (status 10))
 (segment (start 170.18 99.568) (end 162.56 107.188) (width 0.25) (layer B.Cu) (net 10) (status 20))
 (segment (start 181.864 99.568) (end 170.18 99.568) (width 0.25) (layer B.Cu) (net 10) (status 10))
 (segment (start 175.1584 102.7684) (end 178.1556 102.7684) (width 0.25) (layer F.Cu) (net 11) (status 10))
 (segment (start 178.1556 102.7684) (end 180.34 100.584) (width 0.25) (layer F.Cu) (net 11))
 (segment (start 180.34 84.836) (end 181.864 83.312) (width 0.25) (layer F.Cu) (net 11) (status 20))
 (segment (start 180.34 100.584) (end 180.34 84.836) (width 0.25) (layer F.Cu) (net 11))
 (segment (start 181.864 91.44) (end 183.388 91.44) (width 0.25) (layer F.Cu) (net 3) (status 10))
 (segment (start 183.388 91.44) (end 184.404 92.456) (width 0.25) (layer F.Cu) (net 3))
 (segment (start 184.404 113.284) (end 181.864 115.824) (width 0.25) (layer F.Cu) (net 3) (status 20))
 (segment (start 184.404 92.456) (end 184.404 113.284) (width 0.25) (layer F.Cu) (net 3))
 (segment (start 114.808 114.808) (end 119.38 114.808) (width 0.25) (layer F.Cu) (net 3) (status 10))
 (segment (start 119.38 114.808) (end 128.524 105.664) (width 0.25) (layer F.Cu) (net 3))
 (segment (start 135.636 105.664) (end 137.16 107.188) (width 0.25) (layer F.Cu) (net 3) (status 20))
 (segment (start 128.524 105.664) (end 135.636 105.664) (width 0.25) (layer F.Cu) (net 3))
 (segment (start 145.796 115.824) (end 137.16 107.188) (width 0.25) (layer B.Cu) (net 3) (status 20))
 (segment (start 181.864 115.824) (end 145.796 115.824) (width 0.25) (layer B.Cu) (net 3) (status 10))
 (segment (start 120.65 90.5002) (end 139.1158 90.5002) (width 0.25) (layer F.Cu) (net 12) (status 10))
 (segment (start 154.94 106.3244) (end 154.94 107.188) (width 0.25) (layer F.Cu) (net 12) (status 20))
 (segment (start 139.1158 90.5002) (end 154.94 106.3244) (width 0.25) (layer F.Cu) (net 12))
 (segment (start 182.88 98.044) (end 189.484 91.44) (width 0.25) (layer B.Cu) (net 12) (status 20))
 (segment (start 164.084 98.044) (end 182.88 98.044) (width 0.25) (layer B.Cu) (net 12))
 (segment (start 154.94 107.188) (end 164.084 98.044) (width 0.25) (layer B.Cu) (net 12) (status 10))
 (segment (start 135.7884 85.4964) (end 157.48 107.188) (width 0.25) (layer F.Cu) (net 13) (status 20))
 (segment (start 117.5766 85.4964) (end 135.7884 85.4964) (width 0.25) (layer F.Cu) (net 13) (status 10))
 (segment (start 157.48 107.188) (end 163.576 113.284) (width 0.25) (layer B.Cu) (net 13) (status 10))
 (segment (start 186.944 113.284) (end 189.484 115.824) (width 0.25) (layer B.Cu) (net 13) (status 20))
 (segment (start 163.576 113.284) (end 186.944 113.284) (width 0.25) (layer B.Cu) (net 13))
 (segment (start 134.62 127.508) (end 139.7 122.428) (width 0.25) (layer F.Cu) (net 14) (status 20))
 (segment (start 129.54 127.508) (end 134.62 127.508) (width 0.25) (layer F.Cu) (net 14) (status 10))
 (segment (start 142.24 123.063) (end 142.24 122.428) (width 0.25) (layer F.Cu) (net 15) (status 30))
 (segment (start 137.795 127.508) (end 142.24 123.063) (width 0.25) (layer F.Cu) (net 15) (status 30))
 (segment (start 146.05 123.698) (end 144.78 122.428) (width 0.25) (layer F.Cu) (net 16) (status 20))
 (segment (start 146.05 127.508) (end 146.05 123.698) (width 0.25) (layer F.Cu) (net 16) (status 10))
 (segment (start 148.09363 122.428) (end 147.32 122.428) (width 0.25) (layer F.Cu) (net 17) (status 30))
 (segment (start 153.17363 127.508) (end 148.09363 122.428) (width 0.25) (layer F.Cu) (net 17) (status 20))
 (segment (start 154.305 127.508) (end 153.17363 127.508) (width 0.25) (layer F.Cu) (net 17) (status 10))
 (segment (start 162.56 127) (end 156.972 127) (width 0.25) (layer F.Cu) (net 18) (status 10))
 (segment (start 156.972 127) (end 154.432 124.46) (width 0.25) (layer F.Cu) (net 18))
 (segment (start 151.892 124.46) (end 149.86 122.428) (width 0.25) (layer F.Cu) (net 18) (status 20))
 (segment (start 154.432 124.46) (end 151.892 124.46) (width 0.25) (layer F.Cu) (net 18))
 (segment (start 121.92 105.61955) (end 120.94845 105.61955) (width 0.25) (layer F.Cu) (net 1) (status 10))
 (segment (start 120.94845 105.61955) (end 112.268 114.3) (width 0.25) (layer F.Cu) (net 1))
 (segment (start 112.268 114.3) (end 112.268 119.38) (width 0.25) (layer F.Cu) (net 1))
 (segment (start 112.776 119.888) (end 114.808 119.888) (width 0.25) (layer F.Cu) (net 1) (status 20))
 (segment (start 112.268 119.38) (end 112.776 119.888) (width 0.25) (layer F.Cu) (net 1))
 (segment (start 121.92 142.748) (end 121.92 143.256) (width 0.25) (layer F.Cu) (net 19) (status 30))
 (segment (start 129.54 135.128) (end 121.92 142.748) (width 0.25) (layer F.Cu) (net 19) (status 30))
 (segment (start 146.05 143.002) (end 145.796 143.256) (width 0.25) (layer F.Cu) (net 21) (status 30))
 (segment (start 146.05 135.128) (end 146.05 143.002) (width 0.25) (layer F.Cu) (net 21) (status 30))
 (segment (start 154.305 135.128) (end 159.004 139.827) (width 0.25) (layer F.Cu) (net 23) (status 10))
 (segment (start 159.004 141.986) (end 157.734 143.256) (width 0.25) (layer F.Cu) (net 23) (status 20))
 (segment (start 159.004 139.827) (end 159.004 141.986) (width 0.25) (layer F.Cu) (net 23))
 (segment (start 137.795 139.319) (end 133.858 143.256) (width 0.25) (layer F.Cu) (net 20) (status 20))
 (segment (start 137.795 135.128) (end 137.795 139.319) (width 0.25) (layer F.Cu) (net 20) (status 10))
 (segment (start 169.672 141.732) (end 169.672 142.748) (width 0.25) (layer F.Cu) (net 24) (status 20))
 (segment (start 162.56 134.62) (end 169.672 141.732) (width 0.25) (layer F.Cu) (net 24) (status 10))
 (segment (start 121.92 103.67645) (end 128.98755 103.67645) (width 0.25) (layer F.Cu) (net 22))
 (segment (start 128.98755 103.67645) (end 132.08 100.584) (width 0.25) (layer F.Cu) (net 22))
 (segment (start 132.08 100.584) (end 132.08 100.584) (width 0.25) (layer F.Cu) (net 22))
 (via (at 132.08 100.584) (size 0.8) (drill 0.4) (layers F.Cu B.Cu) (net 22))
 (segment (start 132.08 100.584) (end 151.892 80.772) (width 0.25) (layer B.Cu) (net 22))
 (segment (start 151.892 77.6402) (end 152.5854 76.9468) (width 0.25) (layer B.Cu) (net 22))
 (segment (start 151.892 80.772) (end 151.892 77.6402) (width 0.25) (layer B.Cu) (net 22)))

